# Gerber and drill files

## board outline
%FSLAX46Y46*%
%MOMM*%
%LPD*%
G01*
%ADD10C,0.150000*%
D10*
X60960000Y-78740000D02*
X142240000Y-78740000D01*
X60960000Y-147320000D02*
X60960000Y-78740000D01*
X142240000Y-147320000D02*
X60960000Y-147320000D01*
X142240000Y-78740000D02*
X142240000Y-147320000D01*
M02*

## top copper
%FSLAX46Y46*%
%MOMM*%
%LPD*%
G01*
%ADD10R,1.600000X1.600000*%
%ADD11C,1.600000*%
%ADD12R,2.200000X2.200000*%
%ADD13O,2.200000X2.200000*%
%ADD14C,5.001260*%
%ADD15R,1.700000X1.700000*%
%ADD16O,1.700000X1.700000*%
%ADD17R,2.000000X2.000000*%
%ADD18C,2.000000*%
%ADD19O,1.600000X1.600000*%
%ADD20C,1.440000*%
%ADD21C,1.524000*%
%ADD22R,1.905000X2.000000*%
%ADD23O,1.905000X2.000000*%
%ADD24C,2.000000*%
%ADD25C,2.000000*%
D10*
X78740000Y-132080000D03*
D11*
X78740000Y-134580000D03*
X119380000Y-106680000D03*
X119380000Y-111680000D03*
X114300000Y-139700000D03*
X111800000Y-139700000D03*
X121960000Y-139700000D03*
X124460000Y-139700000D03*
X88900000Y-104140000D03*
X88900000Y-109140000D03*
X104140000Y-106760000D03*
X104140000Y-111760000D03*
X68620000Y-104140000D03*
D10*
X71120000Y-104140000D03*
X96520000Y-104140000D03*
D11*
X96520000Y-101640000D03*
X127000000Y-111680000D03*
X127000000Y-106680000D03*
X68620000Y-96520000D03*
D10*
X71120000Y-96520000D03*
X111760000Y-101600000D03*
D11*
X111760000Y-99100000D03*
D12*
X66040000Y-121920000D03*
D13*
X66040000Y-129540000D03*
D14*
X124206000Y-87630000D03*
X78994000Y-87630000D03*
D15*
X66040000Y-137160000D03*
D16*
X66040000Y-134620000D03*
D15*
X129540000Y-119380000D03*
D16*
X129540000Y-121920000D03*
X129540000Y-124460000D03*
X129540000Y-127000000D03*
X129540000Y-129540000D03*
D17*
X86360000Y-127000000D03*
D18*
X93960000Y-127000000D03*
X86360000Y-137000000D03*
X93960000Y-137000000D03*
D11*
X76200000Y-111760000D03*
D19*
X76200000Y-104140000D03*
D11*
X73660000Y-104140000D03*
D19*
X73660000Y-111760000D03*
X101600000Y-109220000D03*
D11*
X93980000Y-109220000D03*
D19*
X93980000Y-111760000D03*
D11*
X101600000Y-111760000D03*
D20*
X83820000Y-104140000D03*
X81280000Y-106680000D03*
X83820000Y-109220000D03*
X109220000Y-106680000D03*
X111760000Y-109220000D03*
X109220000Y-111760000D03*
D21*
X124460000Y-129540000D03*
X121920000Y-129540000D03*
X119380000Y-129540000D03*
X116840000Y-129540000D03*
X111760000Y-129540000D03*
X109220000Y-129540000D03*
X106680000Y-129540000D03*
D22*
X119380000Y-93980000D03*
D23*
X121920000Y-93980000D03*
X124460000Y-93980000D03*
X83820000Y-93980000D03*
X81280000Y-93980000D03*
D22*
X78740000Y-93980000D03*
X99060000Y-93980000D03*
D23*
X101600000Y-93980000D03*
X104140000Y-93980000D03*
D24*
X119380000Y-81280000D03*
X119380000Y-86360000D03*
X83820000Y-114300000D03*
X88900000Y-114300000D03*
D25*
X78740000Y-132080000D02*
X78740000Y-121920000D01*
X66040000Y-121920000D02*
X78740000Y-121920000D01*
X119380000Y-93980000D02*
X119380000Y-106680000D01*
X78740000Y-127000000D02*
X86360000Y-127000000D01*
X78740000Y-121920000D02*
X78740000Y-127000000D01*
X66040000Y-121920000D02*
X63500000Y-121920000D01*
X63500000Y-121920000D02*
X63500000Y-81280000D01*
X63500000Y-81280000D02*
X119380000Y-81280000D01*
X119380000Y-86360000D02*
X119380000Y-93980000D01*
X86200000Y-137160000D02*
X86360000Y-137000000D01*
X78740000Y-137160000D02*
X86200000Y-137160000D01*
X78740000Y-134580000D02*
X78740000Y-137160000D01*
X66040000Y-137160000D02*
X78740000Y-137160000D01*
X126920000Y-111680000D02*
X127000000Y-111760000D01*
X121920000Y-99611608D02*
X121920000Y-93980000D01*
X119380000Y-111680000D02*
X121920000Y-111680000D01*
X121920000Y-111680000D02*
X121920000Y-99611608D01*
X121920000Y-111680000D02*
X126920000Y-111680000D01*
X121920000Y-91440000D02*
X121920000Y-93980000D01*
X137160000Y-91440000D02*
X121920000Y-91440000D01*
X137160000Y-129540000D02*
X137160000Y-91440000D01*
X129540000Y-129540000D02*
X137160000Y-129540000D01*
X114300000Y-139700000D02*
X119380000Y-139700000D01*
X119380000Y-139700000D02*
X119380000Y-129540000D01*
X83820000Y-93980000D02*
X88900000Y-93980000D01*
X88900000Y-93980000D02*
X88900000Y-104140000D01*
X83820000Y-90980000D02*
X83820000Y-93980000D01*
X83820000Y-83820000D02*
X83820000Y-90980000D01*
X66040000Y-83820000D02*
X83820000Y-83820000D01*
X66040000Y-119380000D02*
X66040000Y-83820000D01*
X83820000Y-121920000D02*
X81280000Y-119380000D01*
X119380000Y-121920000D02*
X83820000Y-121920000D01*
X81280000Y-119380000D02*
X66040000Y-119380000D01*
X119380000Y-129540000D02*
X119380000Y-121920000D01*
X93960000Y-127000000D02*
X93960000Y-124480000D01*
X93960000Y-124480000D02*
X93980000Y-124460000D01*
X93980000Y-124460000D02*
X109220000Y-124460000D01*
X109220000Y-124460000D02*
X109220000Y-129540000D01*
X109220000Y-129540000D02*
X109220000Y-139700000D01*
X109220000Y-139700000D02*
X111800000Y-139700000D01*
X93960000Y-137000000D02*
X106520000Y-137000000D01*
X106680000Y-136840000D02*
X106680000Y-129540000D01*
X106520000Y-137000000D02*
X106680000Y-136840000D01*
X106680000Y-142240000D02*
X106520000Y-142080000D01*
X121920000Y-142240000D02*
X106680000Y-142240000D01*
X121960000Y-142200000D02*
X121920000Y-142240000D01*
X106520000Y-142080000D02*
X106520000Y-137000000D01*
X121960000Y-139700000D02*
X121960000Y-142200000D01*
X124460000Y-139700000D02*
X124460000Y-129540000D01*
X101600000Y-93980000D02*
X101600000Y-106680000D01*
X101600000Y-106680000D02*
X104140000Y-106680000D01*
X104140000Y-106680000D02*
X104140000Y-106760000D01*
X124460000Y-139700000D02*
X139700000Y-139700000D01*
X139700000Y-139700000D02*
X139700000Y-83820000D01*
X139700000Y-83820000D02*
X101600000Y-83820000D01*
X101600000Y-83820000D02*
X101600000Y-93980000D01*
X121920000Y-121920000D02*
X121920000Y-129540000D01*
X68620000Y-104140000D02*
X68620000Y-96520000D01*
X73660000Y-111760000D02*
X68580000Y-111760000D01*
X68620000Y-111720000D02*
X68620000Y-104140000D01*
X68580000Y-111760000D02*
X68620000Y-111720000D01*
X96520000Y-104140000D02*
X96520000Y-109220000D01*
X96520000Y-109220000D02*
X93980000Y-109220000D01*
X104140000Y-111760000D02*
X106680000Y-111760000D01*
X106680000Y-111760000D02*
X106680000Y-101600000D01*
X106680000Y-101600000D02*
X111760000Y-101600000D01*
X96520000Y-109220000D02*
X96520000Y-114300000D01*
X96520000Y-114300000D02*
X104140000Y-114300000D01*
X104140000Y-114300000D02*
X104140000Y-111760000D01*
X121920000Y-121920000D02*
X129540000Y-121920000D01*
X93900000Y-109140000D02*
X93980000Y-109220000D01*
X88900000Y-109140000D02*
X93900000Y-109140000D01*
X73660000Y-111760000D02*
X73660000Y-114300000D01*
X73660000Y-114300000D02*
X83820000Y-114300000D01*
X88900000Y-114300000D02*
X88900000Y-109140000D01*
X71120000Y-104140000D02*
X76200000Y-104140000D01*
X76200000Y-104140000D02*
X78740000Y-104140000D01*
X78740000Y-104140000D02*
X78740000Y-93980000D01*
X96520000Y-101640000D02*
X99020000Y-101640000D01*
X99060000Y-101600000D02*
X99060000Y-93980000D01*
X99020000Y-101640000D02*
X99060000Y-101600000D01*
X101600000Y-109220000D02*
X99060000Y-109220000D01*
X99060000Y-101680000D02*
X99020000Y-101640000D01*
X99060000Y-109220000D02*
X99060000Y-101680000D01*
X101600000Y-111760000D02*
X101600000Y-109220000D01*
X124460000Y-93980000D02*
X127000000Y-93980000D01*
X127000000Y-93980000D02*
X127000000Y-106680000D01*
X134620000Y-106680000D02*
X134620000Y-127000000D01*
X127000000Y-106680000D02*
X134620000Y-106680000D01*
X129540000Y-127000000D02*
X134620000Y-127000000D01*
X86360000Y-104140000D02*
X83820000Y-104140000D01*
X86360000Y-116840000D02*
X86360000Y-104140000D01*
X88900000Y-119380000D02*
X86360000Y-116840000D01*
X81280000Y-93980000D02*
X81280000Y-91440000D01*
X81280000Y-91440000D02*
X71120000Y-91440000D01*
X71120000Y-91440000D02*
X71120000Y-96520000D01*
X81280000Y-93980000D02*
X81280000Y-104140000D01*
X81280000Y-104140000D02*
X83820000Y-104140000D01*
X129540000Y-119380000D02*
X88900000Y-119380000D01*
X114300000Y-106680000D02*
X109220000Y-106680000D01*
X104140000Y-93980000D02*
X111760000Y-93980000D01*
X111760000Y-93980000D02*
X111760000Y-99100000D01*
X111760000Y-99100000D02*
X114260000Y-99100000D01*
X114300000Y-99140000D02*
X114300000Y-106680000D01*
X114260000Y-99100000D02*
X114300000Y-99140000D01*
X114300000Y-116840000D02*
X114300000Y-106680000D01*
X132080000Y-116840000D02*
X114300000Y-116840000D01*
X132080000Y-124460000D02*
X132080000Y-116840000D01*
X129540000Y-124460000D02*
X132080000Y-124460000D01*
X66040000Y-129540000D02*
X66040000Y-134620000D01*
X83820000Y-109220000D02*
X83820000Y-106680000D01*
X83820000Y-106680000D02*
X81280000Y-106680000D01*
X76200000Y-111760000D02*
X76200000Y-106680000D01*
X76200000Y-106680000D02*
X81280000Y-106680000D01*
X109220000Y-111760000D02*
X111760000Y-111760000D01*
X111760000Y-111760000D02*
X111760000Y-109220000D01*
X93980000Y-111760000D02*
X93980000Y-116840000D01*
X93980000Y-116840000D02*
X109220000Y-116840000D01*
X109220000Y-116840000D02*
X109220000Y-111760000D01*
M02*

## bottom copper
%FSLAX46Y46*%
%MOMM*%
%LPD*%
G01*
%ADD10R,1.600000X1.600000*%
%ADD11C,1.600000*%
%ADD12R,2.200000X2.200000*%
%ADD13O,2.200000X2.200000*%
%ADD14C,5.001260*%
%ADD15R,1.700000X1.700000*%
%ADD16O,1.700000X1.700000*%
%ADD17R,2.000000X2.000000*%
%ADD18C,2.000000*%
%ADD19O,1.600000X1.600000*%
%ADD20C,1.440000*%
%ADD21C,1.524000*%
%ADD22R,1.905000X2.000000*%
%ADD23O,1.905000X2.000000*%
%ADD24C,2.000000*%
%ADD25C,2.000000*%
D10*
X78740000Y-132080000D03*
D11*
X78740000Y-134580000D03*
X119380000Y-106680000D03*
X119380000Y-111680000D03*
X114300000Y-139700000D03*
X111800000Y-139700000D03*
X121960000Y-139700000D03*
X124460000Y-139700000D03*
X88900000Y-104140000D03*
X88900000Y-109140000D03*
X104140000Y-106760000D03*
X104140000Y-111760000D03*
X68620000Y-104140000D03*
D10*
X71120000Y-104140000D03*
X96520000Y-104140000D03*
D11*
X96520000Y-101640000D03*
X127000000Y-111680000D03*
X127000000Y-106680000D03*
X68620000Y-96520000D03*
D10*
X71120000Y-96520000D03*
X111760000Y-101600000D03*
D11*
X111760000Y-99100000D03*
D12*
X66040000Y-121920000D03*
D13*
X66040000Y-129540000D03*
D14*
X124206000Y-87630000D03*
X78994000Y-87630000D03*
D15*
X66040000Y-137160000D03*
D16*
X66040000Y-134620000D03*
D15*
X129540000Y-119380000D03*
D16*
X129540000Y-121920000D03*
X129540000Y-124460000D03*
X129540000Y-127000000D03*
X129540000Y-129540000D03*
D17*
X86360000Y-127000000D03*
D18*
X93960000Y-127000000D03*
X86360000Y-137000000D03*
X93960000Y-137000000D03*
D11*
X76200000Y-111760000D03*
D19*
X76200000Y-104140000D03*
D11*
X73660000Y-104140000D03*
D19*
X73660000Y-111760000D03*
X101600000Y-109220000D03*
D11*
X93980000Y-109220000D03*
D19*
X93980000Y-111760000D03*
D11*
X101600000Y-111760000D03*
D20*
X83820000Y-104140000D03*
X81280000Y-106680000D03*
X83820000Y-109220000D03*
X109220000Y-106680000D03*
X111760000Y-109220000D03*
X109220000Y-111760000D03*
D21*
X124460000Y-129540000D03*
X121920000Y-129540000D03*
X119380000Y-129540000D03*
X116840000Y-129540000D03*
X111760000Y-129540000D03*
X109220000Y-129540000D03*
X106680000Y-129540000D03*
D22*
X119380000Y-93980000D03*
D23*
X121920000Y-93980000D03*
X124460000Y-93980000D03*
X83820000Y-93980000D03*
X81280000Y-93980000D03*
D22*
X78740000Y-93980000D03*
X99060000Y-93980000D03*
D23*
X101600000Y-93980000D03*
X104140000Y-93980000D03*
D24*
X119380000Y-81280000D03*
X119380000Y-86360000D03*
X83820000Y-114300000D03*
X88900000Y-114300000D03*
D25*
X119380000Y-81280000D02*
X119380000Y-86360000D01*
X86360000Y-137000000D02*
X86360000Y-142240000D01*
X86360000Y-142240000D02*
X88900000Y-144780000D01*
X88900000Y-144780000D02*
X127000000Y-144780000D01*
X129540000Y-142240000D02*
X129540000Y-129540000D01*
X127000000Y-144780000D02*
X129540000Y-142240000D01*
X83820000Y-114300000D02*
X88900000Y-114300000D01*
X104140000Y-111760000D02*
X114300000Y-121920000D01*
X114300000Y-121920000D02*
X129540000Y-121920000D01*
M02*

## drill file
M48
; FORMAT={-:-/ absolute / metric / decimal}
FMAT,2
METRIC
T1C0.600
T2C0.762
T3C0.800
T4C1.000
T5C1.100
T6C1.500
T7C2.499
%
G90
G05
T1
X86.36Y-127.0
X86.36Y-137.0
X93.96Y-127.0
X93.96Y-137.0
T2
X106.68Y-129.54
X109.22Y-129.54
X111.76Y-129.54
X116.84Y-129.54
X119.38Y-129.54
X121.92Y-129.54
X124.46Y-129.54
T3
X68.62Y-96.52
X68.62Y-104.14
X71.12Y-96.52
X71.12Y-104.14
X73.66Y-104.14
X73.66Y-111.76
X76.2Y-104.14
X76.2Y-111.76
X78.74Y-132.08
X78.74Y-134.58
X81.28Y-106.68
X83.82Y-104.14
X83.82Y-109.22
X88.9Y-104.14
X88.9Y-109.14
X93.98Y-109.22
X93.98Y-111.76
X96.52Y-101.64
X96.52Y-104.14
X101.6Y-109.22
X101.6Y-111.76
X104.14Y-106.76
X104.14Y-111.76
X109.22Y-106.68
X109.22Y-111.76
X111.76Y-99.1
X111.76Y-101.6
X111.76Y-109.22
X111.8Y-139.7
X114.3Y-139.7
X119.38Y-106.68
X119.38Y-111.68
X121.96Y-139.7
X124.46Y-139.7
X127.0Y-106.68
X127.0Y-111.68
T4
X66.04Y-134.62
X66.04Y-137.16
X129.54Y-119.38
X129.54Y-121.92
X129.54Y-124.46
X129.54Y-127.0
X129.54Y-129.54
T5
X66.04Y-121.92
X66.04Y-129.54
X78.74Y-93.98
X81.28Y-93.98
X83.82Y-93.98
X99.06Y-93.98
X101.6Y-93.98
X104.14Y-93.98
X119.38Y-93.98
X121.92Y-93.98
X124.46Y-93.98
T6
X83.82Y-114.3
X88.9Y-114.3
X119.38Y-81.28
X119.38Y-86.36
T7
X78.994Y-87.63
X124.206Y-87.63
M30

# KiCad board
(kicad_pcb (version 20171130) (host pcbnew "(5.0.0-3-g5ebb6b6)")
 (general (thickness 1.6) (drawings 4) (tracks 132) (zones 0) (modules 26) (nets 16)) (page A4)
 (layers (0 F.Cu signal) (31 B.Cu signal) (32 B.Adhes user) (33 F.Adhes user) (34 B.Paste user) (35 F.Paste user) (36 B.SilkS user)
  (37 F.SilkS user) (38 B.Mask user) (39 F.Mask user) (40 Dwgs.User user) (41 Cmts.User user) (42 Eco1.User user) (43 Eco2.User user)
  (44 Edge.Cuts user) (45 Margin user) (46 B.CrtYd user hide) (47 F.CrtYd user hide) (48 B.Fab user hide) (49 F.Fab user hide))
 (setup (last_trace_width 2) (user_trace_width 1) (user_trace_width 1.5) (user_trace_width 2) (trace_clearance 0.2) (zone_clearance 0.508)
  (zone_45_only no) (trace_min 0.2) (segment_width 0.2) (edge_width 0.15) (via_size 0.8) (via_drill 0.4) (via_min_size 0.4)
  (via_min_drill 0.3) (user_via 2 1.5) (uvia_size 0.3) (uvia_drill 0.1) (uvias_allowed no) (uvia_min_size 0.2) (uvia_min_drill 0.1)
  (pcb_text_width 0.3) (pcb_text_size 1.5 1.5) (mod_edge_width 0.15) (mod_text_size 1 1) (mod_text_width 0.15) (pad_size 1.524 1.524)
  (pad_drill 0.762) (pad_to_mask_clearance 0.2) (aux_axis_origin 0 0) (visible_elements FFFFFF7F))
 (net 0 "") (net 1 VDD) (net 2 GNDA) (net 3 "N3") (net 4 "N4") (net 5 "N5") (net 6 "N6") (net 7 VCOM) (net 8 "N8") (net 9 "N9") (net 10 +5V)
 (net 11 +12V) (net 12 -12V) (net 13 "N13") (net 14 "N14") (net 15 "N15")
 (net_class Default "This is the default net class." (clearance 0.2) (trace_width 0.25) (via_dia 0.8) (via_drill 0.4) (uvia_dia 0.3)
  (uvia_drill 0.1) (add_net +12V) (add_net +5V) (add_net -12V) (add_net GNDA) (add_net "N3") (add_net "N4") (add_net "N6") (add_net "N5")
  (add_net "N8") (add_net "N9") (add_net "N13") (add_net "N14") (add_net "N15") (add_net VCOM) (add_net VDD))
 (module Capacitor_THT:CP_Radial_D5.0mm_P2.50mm (layer F.Cu) (at 78.74 132.08 270)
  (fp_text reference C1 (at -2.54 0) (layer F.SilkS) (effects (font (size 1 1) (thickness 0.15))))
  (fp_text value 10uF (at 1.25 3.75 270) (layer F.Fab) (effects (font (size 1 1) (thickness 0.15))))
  (pad 1 thru_hole rect (at 0 0 270) (size 1.6 1.6) (drill 0.8) (layers *.Cu *.Mask) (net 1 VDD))
  (pad 2 thru_hole circle (at 2.5 0 270) (size 1.6 1.6) (drill 0.8) (layers *.Cu *.Mask) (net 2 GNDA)))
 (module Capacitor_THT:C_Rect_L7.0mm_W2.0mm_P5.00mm (layer F.Cu) (at 119.38 106.68 270)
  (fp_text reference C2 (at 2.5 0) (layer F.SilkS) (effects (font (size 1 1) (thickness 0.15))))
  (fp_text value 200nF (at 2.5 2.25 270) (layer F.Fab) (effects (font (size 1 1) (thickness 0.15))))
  (pad 1 thru_hole circle (at 0 0 270) (size 1.6 1.6) (drill 0.8) (layers *.Cu *.Mask) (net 1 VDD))
  (pad 2 thru_hole circle (at 5 0 270) (size 1.6 1.6) (drill 0.8) (layers *.Cu *.Mask) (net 2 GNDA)))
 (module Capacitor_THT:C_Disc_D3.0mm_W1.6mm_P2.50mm (layer F.Cu) (at 114.3 139.7 180)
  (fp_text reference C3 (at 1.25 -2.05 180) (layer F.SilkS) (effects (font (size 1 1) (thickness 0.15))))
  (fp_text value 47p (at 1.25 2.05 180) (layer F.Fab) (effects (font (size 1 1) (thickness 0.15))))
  (pad 1 thru_hole circle (at 0 0 180) (size 1.6 1.6) (drill 0.8) (layers *.Cu *.Mask) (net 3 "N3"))
  (pad 2 thru_hole circle (at 2.5 0 180) (size 1.6 1.6) (drill 0.8) (layers *.Cu *.Mask) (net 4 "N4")))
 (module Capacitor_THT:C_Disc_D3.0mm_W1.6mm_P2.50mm (layer F.Cu) (at 124.46 139.7 180)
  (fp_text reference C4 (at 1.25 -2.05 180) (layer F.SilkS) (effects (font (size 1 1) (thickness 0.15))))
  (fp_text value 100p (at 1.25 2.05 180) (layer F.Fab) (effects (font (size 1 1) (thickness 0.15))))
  (pad 2 thru_hole circle (at 2.5 0 180) (size 1.6 1.6) (drill 0.8) (layers *.Cu *.Mask) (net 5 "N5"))
  (pad 1 thru_hole circle (at 0 0 180) (size 1.6 1.6) (drill 0.8) (layers *.Cu *.Mask) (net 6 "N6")))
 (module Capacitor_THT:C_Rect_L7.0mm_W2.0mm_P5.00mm (layer F.Cu) (at 88.9 104.14 270)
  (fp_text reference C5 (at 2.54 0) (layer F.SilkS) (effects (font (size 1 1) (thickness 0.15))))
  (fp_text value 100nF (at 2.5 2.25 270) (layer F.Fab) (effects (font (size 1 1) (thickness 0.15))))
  (pad 1 thru_hole circle (at 0 0 270) (size 1.6 1.6) (drill 0.8) (layers *.Cu *.Mask) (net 3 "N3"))
  (pad 2 thru_hole circle (at 5 0 270) (size 1.6 1.6) (drill 0.8) (layers *.Cu *.Mask) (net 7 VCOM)))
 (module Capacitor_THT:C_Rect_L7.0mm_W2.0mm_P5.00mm (layer F.Cu) (at 104.14 111.76 90)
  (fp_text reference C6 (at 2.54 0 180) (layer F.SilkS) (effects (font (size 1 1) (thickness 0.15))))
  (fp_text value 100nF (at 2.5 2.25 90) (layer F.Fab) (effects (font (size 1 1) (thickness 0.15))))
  (pad 2 thru_hole circle (at 5 0 90) (size 1.6 1.6) (drill 0.8) (layers *.Cu *.Mask) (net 6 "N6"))
  (pad 1 thru_hole circle (at 0 0 90) (size 1.6 1.6) (drill 0.8) (layers *.Cu *.Mask) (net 7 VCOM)))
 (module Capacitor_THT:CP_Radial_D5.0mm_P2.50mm (layer F.Cu) (at 71.12 104.14 180)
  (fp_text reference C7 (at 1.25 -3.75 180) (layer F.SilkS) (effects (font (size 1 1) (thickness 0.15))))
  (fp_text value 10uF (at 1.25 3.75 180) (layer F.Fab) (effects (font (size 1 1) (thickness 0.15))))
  (pad 2 thru_hole circle (at 2.5 0 180) (size 1.6 1.6) (drill 0.8) (layers *.Cu *.Mask) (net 7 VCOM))
  (pad 1 thru_hole rect (at 0 0 180) (size 1.6 1.6) (drill 0.8) (layers *.Cu *.Mask) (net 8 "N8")))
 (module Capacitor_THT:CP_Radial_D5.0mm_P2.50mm (layer F.Cu) (at 96.52 104.14 90)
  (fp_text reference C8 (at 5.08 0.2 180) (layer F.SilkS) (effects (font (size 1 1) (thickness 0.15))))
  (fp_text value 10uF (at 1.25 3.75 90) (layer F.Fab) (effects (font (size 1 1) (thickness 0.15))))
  (pad 1 thru_hole rect (at 0 0 90) (size 1.6 1.6) (drill 0.8) (layers *.Cu *.Mask) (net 7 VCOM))
  (pad 2 thru_hole circle (at 2.5 0 90) (size 1.6 1.6) (drill 0.8) (layers *.Cu *.Mask) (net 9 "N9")))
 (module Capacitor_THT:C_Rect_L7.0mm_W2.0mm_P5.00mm (layer F.Cu) (at 127 106.68 270)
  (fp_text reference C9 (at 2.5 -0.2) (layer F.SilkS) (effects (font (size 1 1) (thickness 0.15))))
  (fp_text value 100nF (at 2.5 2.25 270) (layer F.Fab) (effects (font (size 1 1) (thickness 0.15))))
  (pad 2 thru_hole circle (at 5 0 270) (size 1.6 1.6) (drill 0.8) (layers *.Cu *.Mask) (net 2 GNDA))
  (pad 1 thru_hole circle (at 0 0 270) (size 1.6 1.6) (drill 0.8) (layers *.Cu *.Mask) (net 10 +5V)))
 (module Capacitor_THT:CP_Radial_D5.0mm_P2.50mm (layer F.Cu) (at 71.12 96.52 180)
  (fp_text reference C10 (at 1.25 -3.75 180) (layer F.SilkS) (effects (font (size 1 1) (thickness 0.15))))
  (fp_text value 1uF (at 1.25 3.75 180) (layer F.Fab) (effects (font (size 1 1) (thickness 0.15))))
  (pad 2 thru_hole circle (at 2.5 0 180) (size 1.6 1.6) (drill 0.8) (layers *.Cu *.Mask) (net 7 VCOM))
  (pad 1 thru_hole rect (at 0 0 180) (size 1.6 1.6) (drill 0.8) (layers *.Cu *.Mask) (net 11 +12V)))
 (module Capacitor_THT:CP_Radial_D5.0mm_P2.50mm (layer F.Cu) (at 111.76 101.6 90)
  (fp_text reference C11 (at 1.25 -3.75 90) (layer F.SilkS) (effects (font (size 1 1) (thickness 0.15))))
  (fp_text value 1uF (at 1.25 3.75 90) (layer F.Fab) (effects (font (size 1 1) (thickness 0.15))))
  (pad 1 thru_hole rect (at 0 0 90) (size 1.6 1.6) (drill 0.8) (layers *.Cu *.Mask) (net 7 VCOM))
  (pad 2 thru_hole circle (at 2.5 0 90) (size 1.6 1.6) (drill 0.8) (layers *.Cu *.Mask) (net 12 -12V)))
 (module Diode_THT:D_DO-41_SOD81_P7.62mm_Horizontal (layer F.Cu) (at 66.04 121.92 270)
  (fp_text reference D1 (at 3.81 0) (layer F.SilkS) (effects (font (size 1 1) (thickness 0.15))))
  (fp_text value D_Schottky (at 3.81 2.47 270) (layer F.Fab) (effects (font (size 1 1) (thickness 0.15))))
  (pad 1 thru_hole rect (at 0 0 270) (size 2.2 2.2) (drill 1.1) (layers *.Cu *.Mask) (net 1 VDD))
  (pad 2 thru_hole oval (at 7.62 0 270) (size 2.2 2.2) (drill 1.1) (layers *.Cu *.Mask) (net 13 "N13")))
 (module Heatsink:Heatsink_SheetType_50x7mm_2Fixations (layer F.Cu) (at 101.6 87.63) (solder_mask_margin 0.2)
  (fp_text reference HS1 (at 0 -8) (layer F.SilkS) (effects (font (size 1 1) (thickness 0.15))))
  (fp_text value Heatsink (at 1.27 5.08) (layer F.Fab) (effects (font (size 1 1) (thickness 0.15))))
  (pad 1 thru_hole circle (at 22.606 0) (size 5.00126 5.00126) (drill 2.49936) (layers *.Cu *.Mask))
  (pad 1 thru_hole circle (at -22.606 0) (size 5.00126 5.00126) (drill 2.49936) (layers *.Cu *.Mask)))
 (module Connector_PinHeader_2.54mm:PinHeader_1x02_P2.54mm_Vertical (layer F.Cu) (at 66.04 137.16 180)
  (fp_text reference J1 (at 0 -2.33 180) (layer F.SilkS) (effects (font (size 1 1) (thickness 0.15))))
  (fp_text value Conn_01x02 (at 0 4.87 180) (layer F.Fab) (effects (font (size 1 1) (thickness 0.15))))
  (pad 1 thru_hole rect (at 0 0 180) (size 1.7 1.7) (drill 1) (layers *.Cu *.Mask) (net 2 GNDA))
  (pad 2 thru_hole oval (at 0 2.54 180) (size 1.7 1.7) (drill 1) (layers *.Cu *.Mask) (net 13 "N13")))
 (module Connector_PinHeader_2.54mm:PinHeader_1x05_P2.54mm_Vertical (layer F.Cu) (at 129.54 119.38)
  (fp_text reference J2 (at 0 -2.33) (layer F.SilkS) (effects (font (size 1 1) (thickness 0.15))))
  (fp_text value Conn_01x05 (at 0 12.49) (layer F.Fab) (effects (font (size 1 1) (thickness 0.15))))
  (pad 1 thru_hole rect (at 0 0) (size 1.7 1.7) (drill 1) (layers *.Cu *.Mask) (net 11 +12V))
  (pad 2 thru_hole oval (at 0 2.54) (size 1.7 1.7) (drill 1) (layers *.Cu *.Mask) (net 7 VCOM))
  (pad 3 thru_hole oval (at 0 5.08) (size 1.7 1.7) (drill 1) (layers *.Cu *.Mask) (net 12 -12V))
  (pad 4 thru_hole oval (at 0 7.62) (size 1.7 1.7) (drill 1) (layers *.Cu *.Mask) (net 10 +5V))
  (pad 5 thru_hole oval (at 0 10.16) (size 1.7 1.7) (drill 1) (layers *.Cu *.Mask) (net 2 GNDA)))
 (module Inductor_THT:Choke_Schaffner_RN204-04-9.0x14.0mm (layer F.Cu) (at 86.36 127)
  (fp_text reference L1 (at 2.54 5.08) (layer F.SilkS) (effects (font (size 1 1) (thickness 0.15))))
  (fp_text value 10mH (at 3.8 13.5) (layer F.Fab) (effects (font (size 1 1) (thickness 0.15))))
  (pad 1 thru_hole rect (at 0 0) (size 2 2) (drill 0.6) (layers *.Cu *.Mask) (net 1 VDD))
  (pad 2 thru_hole circle (at 7.6 0) (size 2 2) (drill 0.6) (layers *.Cu *.Mask) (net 4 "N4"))
  (pad 3 thru_hole circle (at 0 10) (size 2 2) (drill 0.6) (layers *.Cu *.Mask) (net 2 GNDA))
  (pad 4 thru_hole circle (at 7.6 10) (size 2 2) (drill 0.6) (layers *.Cu *.Mask) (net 5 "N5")))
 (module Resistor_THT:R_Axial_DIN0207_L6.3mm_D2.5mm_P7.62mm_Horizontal (layer F.Cu) (at 76.2 111.76 90)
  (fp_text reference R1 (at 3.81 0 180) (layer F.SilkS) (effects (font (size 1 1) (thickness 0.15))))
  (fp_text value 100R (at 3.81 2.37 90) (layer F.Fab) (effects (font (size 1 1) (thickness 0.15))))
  (pad 1 thru_hole circle (at 0 0 90) (size 1.6 1.6) (drill 0.8) (layers *.Cu *.Mask) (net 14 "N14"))
  (pad 2 thru_hole oval (at 7.62 0 90) (size 1.6 1.6) (drill 0.8) (layers *.Cu *.Mask) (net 8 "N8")))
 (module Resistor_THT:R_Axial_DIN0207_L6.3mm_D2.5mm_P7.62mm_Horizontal (layer F.Cu) (at 73.66 104.14 270)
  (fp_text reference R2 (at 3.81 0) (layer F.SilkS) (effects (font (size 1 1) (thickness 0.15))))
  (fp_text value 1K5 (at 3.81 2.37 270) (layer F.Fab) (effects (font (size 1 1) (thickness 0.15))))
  (pad 1 thru_hole circle (at 0 0 270) (size 1.6 1.6) (drill 0.8) (layers *.Cu *.Mask) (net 8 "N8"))
  (pad 2 thru_hole oval (at 7.62 0 270) (size 1.6 1.6) (drill 0.8) (layers *.Cu *.Mask) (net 7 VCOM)))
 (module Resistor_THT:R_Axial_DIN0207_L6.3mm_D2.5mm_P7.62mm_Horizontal (layer F.Cu) (at 93.98 109.22)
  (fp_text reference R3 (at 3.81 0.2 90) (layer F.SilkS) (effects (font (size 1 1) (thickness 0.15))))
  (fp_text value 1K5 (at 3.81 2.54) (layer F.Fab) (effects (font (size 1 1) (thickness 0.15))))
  (pad 2 thru_hole oval (at 7.62 0) (size 1.6 1.6) (drill 0.8) (layers *.Cu *.Mask) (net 9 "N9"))
  (pad 1 thru_hole circle (at 0 0) (size 1.6 1.6) (drill 0.8) (layers *.Cu *.Mask) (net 7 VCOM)))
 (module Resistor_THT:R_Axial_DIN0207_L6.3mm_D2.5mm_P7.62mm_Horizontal (layer F.Cu) (at 101.6 111.76 180)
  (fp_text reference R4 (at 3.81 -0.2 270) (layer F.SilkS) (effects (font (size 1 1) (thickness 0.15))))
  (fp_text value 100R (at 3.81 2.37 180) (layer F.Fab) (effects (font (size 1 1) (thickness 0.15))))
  (pad 2 thru_hole oval (at 7.62 0 180) (size 1.6 1.6) (drill 0.8) (layers *.Cu *.Mask) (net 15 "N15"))
  (pad 1 thru_hole circle (at 0 0 180) (size 1.6 1.6) (drill 0.8) (layers *.Cu *.Mask) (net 9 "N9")))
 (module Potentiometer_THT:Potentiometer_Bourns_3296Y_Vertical (layer F.Cu) (at 83.82 109.22 270)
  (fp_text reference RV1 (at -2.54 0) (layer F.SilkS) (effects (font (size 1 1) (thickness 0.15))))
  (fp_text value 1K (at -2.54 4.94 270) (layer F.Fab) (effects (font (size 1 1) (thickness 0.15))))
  (pad 3 thru_hole circle (at -5.08 0 270) (size 1.44 1.44) (drill 0.8) (layers *.Cu *.Mask) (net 11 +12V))
  (pad 2 thru_hole circle (at -2.54 2.54 270) (size 1.44 1.44) (drill 0.8) (layers *.Cu *.Mask) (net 14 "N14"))
  (pad 1 thru_hole circle (at 0 0 270) (size 1.44 1.44) (drill 0.8) (layers *.Cu *.Mask) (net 14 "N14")))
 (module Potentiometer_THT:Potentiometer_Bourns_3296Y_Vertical (layer F.Cu) (at 109.22 106.68 90)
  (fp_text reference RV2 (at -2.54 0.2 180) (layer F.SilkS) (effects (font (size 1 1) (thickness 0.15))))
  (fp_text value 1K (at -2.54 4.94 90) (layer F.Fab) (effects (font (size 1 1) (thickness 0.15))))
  (pad 1 thru_hole circle (at 0 0 90) (size 1.44 1.44) (drill 0.8) (layers *.Cu *.Mask) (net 12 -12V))
  (pad 2 thru_hole circle (at -2.54 2.54 90) (size 1.44 1.44) (drill 0.8) (layers *.Cu *.Mask) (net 15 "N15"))
  (pad 3 thru_hole circle (at -5.08 0 90) (size 1.44 1.44) (drill 0.8) (layers *.Cu *.Mask) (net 15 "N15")))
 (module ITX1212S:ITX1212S (layer F.Cu) (at 114.3 129.54)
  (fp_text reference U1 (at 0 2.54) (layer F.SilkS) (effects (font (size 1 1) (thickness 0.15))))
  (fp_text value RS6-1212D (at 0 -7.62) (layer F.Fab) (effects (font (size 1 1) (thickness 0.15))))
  (pad 8 thru_hole circle (at 10.16 0) (size 1.524 1.524) (drill 0.762) (layers *.Cu *.Mask) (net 6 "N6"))
  (pad 7 thru_hole circle (at 7.62 0) (size 1.524 1.524) (drill 0.762) (layers *.Cu *.Mask) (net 7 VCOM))
  (pad 6 thru_hole circle (at 5.08 0) (size 1.524 1.524) (drill 0.762) (layers *.Cu *.Mask) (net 3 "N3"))
  (pad 5 thru_hole circle (at 2.54 0) (size 1.524 1.524) (drill 0.762) (layers *.Cu *.Mask))
  (pad 3 thru_hole circle (at -2.54 0) (size 1.524 1.524) (drill 0.762) (layers *.Cu *.Mask))
  (pad 2 thru_hole circle (at -5.08 0) (size 1.524 1.524) (drill 0.762) (layers *.Cu *.Mask) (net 4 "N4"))
  (pad 1 thru_hole circle (at -7.62 0) (size 1.524 1.524) (drill 0.762) (layers *.Cu *.Mask) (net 5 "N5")))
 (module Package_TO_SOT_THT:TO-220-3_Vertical (layer F.Cu) (at 119.38 93.98)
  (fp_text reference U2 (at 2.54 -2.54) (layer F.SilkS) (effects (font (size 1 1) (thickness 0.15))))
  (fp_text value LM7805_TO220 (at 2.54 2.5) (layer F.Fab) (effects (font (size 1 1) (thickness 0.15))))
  (pad 1 thru_hole rect (at 0 0) (size 1.905 2) (drill 1.1) (layers *.Cu *.Mask) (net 1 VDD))
  (pad 2 thru_hole oval (at 2.54 0) (size 1.905 2) (drill 1.1) (layers *.Cu *.Mask) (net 2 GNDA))
  (pad 3 thru_hole oval (at 5.08 0) (size 1.905 2) (drill 1.1) (layers *.Cu *.Mask) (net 10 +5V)))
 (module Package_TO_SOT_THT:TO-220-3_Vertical (layer F.Cu) (at 78.74 93.98)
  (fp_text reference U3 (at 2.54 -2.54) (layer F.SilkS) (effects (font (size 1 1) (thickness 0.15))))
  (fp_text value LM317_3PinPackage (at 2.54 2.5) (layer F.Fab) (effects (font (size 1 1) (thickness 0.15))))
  (pad 3 thru_hole oval (at 5.08 0) (size 1.905 2) (drill 1.1) (layers *.Cu *.Mask) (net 3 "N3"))
  (pad 2 thru_hole oval (at 2.54 0) (size 1.905 2) (drill 1.1) (layers *.Cu *.Mask) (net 11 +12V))
  (pad 1 thru_hole rect (at 0 0) (size 1.905 2) (drill 1.1) (layers *.Cu *.Mask) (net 8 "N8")))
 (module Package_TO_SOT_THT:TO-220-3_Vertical (layer F.Cu) (at 99.06 93.98)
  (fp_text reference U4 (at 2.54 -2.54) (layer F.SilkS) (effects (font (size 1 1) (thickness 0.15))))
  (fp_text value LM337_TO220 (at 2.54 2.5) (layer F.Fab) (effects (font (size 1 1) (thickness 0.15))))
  (pad 1 thru_hole rect (at 0 0) (size 1.905 2) (drill 1.1) (layers *.Cu *.Mask) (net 9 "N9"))
  (pad 2 thru_hole oval (at 2.54 0) (size 1.905 2) (drill 1.1) (layers *.Cu *.Mask) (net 6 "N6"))
  (pad 3 thru_hole oval (at 5.08 0) (size 1.905 2) (drill 1.1) (layers *.Cu *.Mask) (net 12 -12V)))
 (gr_line (start 60.96 78.74) (end 142.24 78.74) (layer Edge.Cuts) (width 0.15))
 (gr_line (start 60.96 147.32) (end 60.96 78.74) (layer Edge.Cuts) (width 0.15))
 (gr_line (start 142.24 147.32) (end 60.96 147.32) (layer Edge.Cuts) (width 0.15))
 (gr_line (start 142.24 78.74) (end 142.24 147.32) (layer Edge.Cuts) (width 0.15))
 (segment (start 78.74 132.08) (end 78.74 121.92) (width 2) (layer F.Cu) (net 1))
 (segment (start 66.04 121.92) (end 78.74 121.92) (width 2) (layer F.Cu) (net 1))
 (segment (start 119.38 93.98) (end 119.38 106.68) (width 2) (layer F.Cu) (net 1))
 (segment (start 78.74 127) (end 86.36 127) (width 2) (layer F.Cu) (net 1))
 (segment (start 78.74 121.92) (end 78.74 127) (width 2) (layer F.Cu) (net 1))
 (segment (start 66.04 121.92) (end 63.5 121.92) (width 2) (layer F.Cu) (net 1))
 (segment (start 63.5 121.92) (end 63.5 81.28) (width 2) (layer F.Cu) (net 1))
 (segment (start 63.5 81.28) (end 119.38 81.28) (width 2) (layer F.Cu) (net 1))
 (via (at 119.38 81.28) (size 2) (drill 1.5) (layers F.Cu B.Cu) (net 1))
 (segment (start 119.38 81.28) (end 119.38 86.36) (width 2) (layer B.Cu) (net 1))
 (via (at 119.38 86.36) (size 2) (drill 1.5) (layers F.Cu B.Cu) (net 1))
 (segment (start 119.38 86.36) (end 119.38 93.98) (width 2) (layer F.Cu) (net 1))
 (segment (start 86.2 137.16) (end 86.36 137) (width 2) (layer F.Cu) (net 2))
 (segment (start 78.74 137.16) (end 86.2 137.16) (width 2) (layer F.Cu) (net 2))
 (segment (start 78.74 134.58) (end 78.74 137.16) (width 2) (layer F.Cu) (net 2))
 (segment (start 66.04 137.16) (end 78.74 137.16) (width 2) (layer F.Cu) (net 2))
 (segment (start 126.92 111.68) (end 127 111.76) (width 2) (layer F.Cu) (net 2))
 (segment (start 121.92 99.611608) (end 121.92 93.98) (width 2) (layer F.Cu) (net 2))
 (segment (start 119.38 111.68) (end 121.92 111.68) (width 2) (layer F.Cu) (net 2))
 (segment (start 121.92 111.68) (end 121.92 99.611608) (width 2) (layer F.Cu) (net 2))
 (segment (start 121.92 111.68) (end 126.92 111.68) (width 2) (layer F.Cu) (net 2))
 (segment (start 121.92 91.44) (end 121.92 93.98) (width 2) (layer F.Cu) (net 2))
 (segment (start 137.16 91.44) (end 121.92 91.44) (width 2) (layer F.Cu) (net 2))
 (segment (start 137.16 129.54) (end 137.16 91.44) (width 2) (layer F.Cu) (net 2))
 (segment (start 129.54 129.54) (end 137.16 129.54) (width 2) (layer F.Cu) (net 2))
 (segment (start 86.36 137) (end 86.36 142.24) (width 2) (layer B.Cu) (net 2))
 (segment (start 86.36 142.24) (end 88.9 144.78) (width 2) (layer B.Cu) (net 2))
 (segment (start 88.9 144.78) (end 127 144.78) (width 2) (layer B.Cu) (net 2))
 (segment (start 129.54 142.24) (end 129.54 129.54) (width 2) (layer B.Cu) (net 2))
 (segment (start 127 144.78) (end 129.54 142.24) (width 2) (layer B.Cu) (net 2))
 (segment (start 114.3 139.7) (end 119.38 139.7) (width 2) (layer F.Cu) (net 3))
 (segment (start 119.38 139.7) (end 119.38 129.54) (width 2) (layer F.Cu) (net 3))
 (segment (start 83.82 93.98) (end 88.9 93.98) (width 2) (layer F.Cu) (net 3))
 (segment (start 88.9 93.98) (end 88.9 104.14) (width 2) (layer F.Cu) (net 3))
 (segment (start 83.82 90.98) (end 83.82 93.98) (width 2) (layer F.Cu) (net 3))
 (segment (start 83.82 83.82) (end 83.82 90.98) (width 2) (layer F.Cu) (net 3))
 (segment (start 66.04 83.82) (end 83.82 83.82) (width 2) (layer F.Cu) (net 3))
 (segment (start 66.04 119.38) (end 66.04 83.82) (width 2) (layer F.Cu) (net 3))
 (segment (start 83.82 121.92) (end 81.28 119.38) (width 2) (layer F.Cu) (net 3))
 (segment (start 119.38 121.92) (end 83.82 121.92) (width 2) (layer F.Cu) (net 3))
 (segment (start 81.28 119.38) (end 66.04 119.38) (width 2) (layer F.Cu) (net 3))
 (segment (start 119.38 129.54) (end 119.38 121.92) (width 2) (layer F.Cu) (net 3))
 (segment (start 93.96 127) (end 93.96 124.48) (width 2) (layer F.Cu) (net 4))
 (segment (start 93.96 124.48) (end 93.98 124.46) (width 2) (layer F.Cu) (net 4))
 (segment (start 93.98 124.46) (end 109.22 124.46) (width 2) (layer F.Cu) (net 4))
 (segment (start 109.22 124.46) (end 109.22 129.54) (width 2) (layer F.Cu) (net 4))
 (segment (start 109.22 129.54) (end 109.22 139.7) (width 2) (layer F.Cu) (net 4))
 (segment (start 109.22 139.7) (end 111.8 139.7) (width 2) (layer F.Cu) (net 4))
 (segment (start 93.96 137) (end 106.52 137) (width 2) (layer F.Cu) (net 5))
 (segment (start 106.68 136.84) (end 106.68 129.54) (width 2) (layer F.Cu) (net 5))
 (segment (start 106.52 137) (end 106.68 136.84) (width 2) (layer F.Cu) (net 5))
 (segment (start 106.68 142.24) (end 106.52 142.08) (width 2) (layer F.Cu) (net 5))
 (segment (start 121.92 142.24) (end 106.68 142.24) (width 2) (layer F.Cu) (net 5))
 (segment (start 121.96 142.2) (end 121.92 142.24) (width 2) (layer F.Cu) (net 5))
 (segment (start 106.52 142.08) (end 106.52 137) (width 2) (layer F.Cu) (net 5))
 (segment (start 121.96 139.7) (end 121.96 142.2) (width 2) (layer F.Cu) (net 5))
 (segment (start 124.46 139.7) (end 124.46 129.54) (width 2) (layer F.Cu) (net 6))
 (segment (start 101.6 93.98) (end 101.6 106.68) (width 2) (layer F.Cu) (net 6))
 (segment (start 101.6 106.68) (end 104.14 106.68) (width 2) (layer F.Cu) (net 6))
 (segment (start 104.14 106.68) (end 104.14 106.76) (width 2) (layer F.Cu) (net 6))
 (segment (start 124.46 139.7) (end 139.7 139.7) (width 2) (layer F.Cu) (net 6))
 (segment (start 139.7 139.7) (end 139.7 83.82) (width 2) (layer F.Cu) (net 6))
 (segment (start 139.7 83.82) (end 101.6 83.82) (width 2) (layer F.Cu) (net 6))
 (segment (start 101.6 83.82) (end 101.6 93.98) (width 2) (layer F.Cu) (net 6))
 (segment (start 121.92 121.92) (end 121.92 129.54) (width 2) (layer F.Cu) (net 7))
 (segment (start 68.62 104.14) (end 68.62 96.52) (width 2) (layer F.Cu) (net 7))
 (segment (start 73.66 111.76) (end 68.58 111.76) (width 2) (layer F.Cu) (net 7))
 (segment (start 68.62 111.72) (end 68.62 104.14) (width 2) (layer F.Cu) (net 7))
 (segment (start 68.58 111.76) (end 68.62 111.72) (width 2) (layer F.Cu) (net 7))
 (segment (start 96.52 104.14) (end 96.52 109.22) (width 2) (layer F.Cu) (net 7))
 (segment (start 96.52 109.22) (end 93.98 109.22) (width 2) (layer F.Cu) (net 7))
 (segment (start 104.14 111.76) (end 106.68 111.76) (width 2) (layer F.Cu) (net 7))
 (segment (start 106.68 111.76) (end 106.68 101.6) (width 2) (layer F.Cu) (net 7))
 (segment (start 106.68 101.6) (end 111.76 101.6) (width 2) (layer F.Cu) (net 7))
 (segment (start 96.52 109.22) (end 96.52 114.3) (width 2) (layer F.Cu) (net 7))
 (segment (start 96.52 114.3) (end 104.14 114.3) (width 2) (layer F.Cu) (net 7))
 (segment (start 104.14 114.3) (end 104.14 111.76) (width 2) (layer F.Cu) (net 7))
 (segment (start 121.92 121.92) (end 129.54 121.92) (width 2) (layer F.Cu) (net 7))
 (segment (start 93.9 109.14) (end 93.98 109.22) (width 2) (layer F.Cu) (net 7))
 (segment (start 88.9 109.14) (end 93.9 109.14) (width 2) (layer F.Cu) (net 7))
 (segment (start 73.66 111.76) (end 73.66 114.3) (width 2) (layer F.Cu) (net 7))
 (segment (start 73.66 114.3) (end 83.82 114.3) (width 2) (layer F.Cu) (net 7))
 (via (at 83.82 114.3) (size 2) (drill 1.5) (layers F.Cu B.Cu) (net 7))
 (segment (start 83.82 114.3) (end 88.9 114.3) (width 2) (layer B.Cu) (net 7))
 (via (at 88.9 114.3) (size 2) (drill 1.5) (layers F.Cu B.Cu) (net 7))
 (segment (start 88.9 114.3) (end 88.9 109.14) (width 2) (layer F.Cu) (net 7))
 (segment (start 104.14 111.76) (end 114.3 121.92) (width 2) (layer B.Cu) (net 7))
 (segment (start 114.3 121.92) (end 129.54 121.92) (width 2) (layer B.Cu) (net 7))
 (segment (start 71.12 104.14) (end 76.2 104.14) (width 2) (layer F.Cu) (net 8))
 (segment (start 76.2 104.14) (end 78.74 104.14) (width 2) (layer F.Cu) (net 8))
 (segment (start 78.74 104.14) (end 78.74 93.98) (width 2) (layer F.Cu) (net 8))
 (segment (start 96.52 101.64) (end 99.02 101.64) (width 2) (layer F.Cu) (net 9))
 (segment (start 99.06 101.6) (end 99.06 93.98) (width 2) (layer F.Cu) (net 9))
 (segment (start 99.02 101.64) (end 99.06 101.6) (width 2) (layer F.Cu) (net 9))
 (segment (start 101.6 109.22) (end 99.06 109.22) (width 2) (layer F.Cu) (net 9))
 (segment (start 99.06 101.68) (end 99.02 101.64) (width 2) (layer F.Cu) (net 9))
 (segment (start 99.06 109.22) (end 99.06 101.68) (width 2) (layer F.Cu) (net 9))
 (segment (start 101.6 111.76) (end 101.6 109.22) (width 2) (layer F.Cu) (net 9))
 (segment (start 124.46 93.98) (end 127 93.98) (width 2) (layer F.Cu) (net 10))
 (segment (start 127 93.98) (end 127 106.68) (width 2) (layer F.Cu) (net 10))
 (segment (start 134.62 106.68) (end 134.62 127) (width 2) (layer F.Cu) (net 10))
 (segment (start 127 106.68) (end 134.62 106.68) (width 2) (layer F.Cu) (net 10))
 (segment (start 129.54 127) (end 134.62 127) (width 2) (layer F.Cu) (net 10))
 (segment (start 86.36 104.14) (end 83.82 104.14) (width 2) (layer F.Cu) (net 11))
 (segment (start 86.36 116.84) (end 86.36 104.14) (width 2) (layer F.Cu) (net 11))
 (segment (start 88.9 119.38) (end 86.36 116.84) (width 2) (layer F.Cu) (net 11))
 (segment (start 81.28 93.98) (end 81.28 91.44) (width 2) (layer F.Cu) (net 11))
 (segment (start 81.28 91.44) (end 71.12 91.44) (width 2) (layer F.Cu) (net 11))
 (segment (start 71.12 91.44) (end 71.12 96.52) (width 2) (layer F.Cu) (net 11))
 (segment (start 81.28 93.98) (end 81.28 104.14) (width 2) (layer F.Cu) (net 11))
 (segment (start 81.28 104.14) (end 83.82 104.14) (width 2) (layer F.Cu) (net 11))
 (segment (start 129.54 119.38) (end 88.9 119.38) (width 2) (layer F.Cu) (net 11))
 (segment (start 114.3 106.68) (end 109.22 106.68) (width 2) (layer F.Cu) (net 12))
 (segment (start 104.14 93.98) (end 111.76 93.98) (width 2) (layer F.Cu) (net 12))
 (segment (start 111.76 93.98) (end 111.76 99.1) (width 2) (layer F.Cu) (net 12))
 (segment (start 111.76 99.1) (end 114.26 99.1) (width 2) (layer F.Cu) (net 12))
 (segment (start 114.3 99.14) (end 114.3 106.68) (width 2) (layer F.Cu) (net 12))
 (segment (start 114.26 99.1) (end 114.3 99.14) (width 2) (layer F.Cu) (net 12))
 (segment (start 114.3 116.84) (end 114.3 106.68) (width 2) (layer F.Cu) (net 12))
 (segment (start 132.08 116.84) (end 114.3 116.84) (width 2) (layer F.Cu) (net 12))
 (segment (start 132.08 124.46) (end 132.08 116.84) (width 2) (layer F.Cu) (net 12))
 (segment (start 129.54 124.46) (end 132.08 124.46) (width 2) (layer F.Cu) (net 12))
 (segment (start 66.04 129.54) (end 66.04 134.62) (width 2) (layer F.Cu) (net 13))
 (segment (start 83.82 109.22) (end 83.82 106.68) (width 2) (layer F.Cu) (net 14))
 (segment (start 83.82 106.68) (end 81.28 106.68) (width 2) (layer F.Cu) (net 14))
 (segment (start 76.2 111.76) (end 76.2 106.68) (width 2) (layer F.Cu) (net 14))
 (segment (start 76.2 106.68) (end 81.28 106.68) (width 2) (layer F.Cu) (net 14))
 (segment (start 109.22 111.76) (end 111.76 111.76) (width 2) (layer F.Cu) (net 15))
 (segment (start 111.76 111.76) (end 111.76 109.22) (width 2) (layer F.Cu) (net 15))
 (segment (start 93.98 111.76) (end 93.98 116.84) (width 2) (layer F.Cu) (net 15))
 (segment (start 93.98 116.84) (end 109.22 116.84) (width 2) (layer F.Cu) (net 15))
 (segment (start 109.22 116.84) (end 109.22 111.76) (width 2) (layer F.Cu) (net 15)))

